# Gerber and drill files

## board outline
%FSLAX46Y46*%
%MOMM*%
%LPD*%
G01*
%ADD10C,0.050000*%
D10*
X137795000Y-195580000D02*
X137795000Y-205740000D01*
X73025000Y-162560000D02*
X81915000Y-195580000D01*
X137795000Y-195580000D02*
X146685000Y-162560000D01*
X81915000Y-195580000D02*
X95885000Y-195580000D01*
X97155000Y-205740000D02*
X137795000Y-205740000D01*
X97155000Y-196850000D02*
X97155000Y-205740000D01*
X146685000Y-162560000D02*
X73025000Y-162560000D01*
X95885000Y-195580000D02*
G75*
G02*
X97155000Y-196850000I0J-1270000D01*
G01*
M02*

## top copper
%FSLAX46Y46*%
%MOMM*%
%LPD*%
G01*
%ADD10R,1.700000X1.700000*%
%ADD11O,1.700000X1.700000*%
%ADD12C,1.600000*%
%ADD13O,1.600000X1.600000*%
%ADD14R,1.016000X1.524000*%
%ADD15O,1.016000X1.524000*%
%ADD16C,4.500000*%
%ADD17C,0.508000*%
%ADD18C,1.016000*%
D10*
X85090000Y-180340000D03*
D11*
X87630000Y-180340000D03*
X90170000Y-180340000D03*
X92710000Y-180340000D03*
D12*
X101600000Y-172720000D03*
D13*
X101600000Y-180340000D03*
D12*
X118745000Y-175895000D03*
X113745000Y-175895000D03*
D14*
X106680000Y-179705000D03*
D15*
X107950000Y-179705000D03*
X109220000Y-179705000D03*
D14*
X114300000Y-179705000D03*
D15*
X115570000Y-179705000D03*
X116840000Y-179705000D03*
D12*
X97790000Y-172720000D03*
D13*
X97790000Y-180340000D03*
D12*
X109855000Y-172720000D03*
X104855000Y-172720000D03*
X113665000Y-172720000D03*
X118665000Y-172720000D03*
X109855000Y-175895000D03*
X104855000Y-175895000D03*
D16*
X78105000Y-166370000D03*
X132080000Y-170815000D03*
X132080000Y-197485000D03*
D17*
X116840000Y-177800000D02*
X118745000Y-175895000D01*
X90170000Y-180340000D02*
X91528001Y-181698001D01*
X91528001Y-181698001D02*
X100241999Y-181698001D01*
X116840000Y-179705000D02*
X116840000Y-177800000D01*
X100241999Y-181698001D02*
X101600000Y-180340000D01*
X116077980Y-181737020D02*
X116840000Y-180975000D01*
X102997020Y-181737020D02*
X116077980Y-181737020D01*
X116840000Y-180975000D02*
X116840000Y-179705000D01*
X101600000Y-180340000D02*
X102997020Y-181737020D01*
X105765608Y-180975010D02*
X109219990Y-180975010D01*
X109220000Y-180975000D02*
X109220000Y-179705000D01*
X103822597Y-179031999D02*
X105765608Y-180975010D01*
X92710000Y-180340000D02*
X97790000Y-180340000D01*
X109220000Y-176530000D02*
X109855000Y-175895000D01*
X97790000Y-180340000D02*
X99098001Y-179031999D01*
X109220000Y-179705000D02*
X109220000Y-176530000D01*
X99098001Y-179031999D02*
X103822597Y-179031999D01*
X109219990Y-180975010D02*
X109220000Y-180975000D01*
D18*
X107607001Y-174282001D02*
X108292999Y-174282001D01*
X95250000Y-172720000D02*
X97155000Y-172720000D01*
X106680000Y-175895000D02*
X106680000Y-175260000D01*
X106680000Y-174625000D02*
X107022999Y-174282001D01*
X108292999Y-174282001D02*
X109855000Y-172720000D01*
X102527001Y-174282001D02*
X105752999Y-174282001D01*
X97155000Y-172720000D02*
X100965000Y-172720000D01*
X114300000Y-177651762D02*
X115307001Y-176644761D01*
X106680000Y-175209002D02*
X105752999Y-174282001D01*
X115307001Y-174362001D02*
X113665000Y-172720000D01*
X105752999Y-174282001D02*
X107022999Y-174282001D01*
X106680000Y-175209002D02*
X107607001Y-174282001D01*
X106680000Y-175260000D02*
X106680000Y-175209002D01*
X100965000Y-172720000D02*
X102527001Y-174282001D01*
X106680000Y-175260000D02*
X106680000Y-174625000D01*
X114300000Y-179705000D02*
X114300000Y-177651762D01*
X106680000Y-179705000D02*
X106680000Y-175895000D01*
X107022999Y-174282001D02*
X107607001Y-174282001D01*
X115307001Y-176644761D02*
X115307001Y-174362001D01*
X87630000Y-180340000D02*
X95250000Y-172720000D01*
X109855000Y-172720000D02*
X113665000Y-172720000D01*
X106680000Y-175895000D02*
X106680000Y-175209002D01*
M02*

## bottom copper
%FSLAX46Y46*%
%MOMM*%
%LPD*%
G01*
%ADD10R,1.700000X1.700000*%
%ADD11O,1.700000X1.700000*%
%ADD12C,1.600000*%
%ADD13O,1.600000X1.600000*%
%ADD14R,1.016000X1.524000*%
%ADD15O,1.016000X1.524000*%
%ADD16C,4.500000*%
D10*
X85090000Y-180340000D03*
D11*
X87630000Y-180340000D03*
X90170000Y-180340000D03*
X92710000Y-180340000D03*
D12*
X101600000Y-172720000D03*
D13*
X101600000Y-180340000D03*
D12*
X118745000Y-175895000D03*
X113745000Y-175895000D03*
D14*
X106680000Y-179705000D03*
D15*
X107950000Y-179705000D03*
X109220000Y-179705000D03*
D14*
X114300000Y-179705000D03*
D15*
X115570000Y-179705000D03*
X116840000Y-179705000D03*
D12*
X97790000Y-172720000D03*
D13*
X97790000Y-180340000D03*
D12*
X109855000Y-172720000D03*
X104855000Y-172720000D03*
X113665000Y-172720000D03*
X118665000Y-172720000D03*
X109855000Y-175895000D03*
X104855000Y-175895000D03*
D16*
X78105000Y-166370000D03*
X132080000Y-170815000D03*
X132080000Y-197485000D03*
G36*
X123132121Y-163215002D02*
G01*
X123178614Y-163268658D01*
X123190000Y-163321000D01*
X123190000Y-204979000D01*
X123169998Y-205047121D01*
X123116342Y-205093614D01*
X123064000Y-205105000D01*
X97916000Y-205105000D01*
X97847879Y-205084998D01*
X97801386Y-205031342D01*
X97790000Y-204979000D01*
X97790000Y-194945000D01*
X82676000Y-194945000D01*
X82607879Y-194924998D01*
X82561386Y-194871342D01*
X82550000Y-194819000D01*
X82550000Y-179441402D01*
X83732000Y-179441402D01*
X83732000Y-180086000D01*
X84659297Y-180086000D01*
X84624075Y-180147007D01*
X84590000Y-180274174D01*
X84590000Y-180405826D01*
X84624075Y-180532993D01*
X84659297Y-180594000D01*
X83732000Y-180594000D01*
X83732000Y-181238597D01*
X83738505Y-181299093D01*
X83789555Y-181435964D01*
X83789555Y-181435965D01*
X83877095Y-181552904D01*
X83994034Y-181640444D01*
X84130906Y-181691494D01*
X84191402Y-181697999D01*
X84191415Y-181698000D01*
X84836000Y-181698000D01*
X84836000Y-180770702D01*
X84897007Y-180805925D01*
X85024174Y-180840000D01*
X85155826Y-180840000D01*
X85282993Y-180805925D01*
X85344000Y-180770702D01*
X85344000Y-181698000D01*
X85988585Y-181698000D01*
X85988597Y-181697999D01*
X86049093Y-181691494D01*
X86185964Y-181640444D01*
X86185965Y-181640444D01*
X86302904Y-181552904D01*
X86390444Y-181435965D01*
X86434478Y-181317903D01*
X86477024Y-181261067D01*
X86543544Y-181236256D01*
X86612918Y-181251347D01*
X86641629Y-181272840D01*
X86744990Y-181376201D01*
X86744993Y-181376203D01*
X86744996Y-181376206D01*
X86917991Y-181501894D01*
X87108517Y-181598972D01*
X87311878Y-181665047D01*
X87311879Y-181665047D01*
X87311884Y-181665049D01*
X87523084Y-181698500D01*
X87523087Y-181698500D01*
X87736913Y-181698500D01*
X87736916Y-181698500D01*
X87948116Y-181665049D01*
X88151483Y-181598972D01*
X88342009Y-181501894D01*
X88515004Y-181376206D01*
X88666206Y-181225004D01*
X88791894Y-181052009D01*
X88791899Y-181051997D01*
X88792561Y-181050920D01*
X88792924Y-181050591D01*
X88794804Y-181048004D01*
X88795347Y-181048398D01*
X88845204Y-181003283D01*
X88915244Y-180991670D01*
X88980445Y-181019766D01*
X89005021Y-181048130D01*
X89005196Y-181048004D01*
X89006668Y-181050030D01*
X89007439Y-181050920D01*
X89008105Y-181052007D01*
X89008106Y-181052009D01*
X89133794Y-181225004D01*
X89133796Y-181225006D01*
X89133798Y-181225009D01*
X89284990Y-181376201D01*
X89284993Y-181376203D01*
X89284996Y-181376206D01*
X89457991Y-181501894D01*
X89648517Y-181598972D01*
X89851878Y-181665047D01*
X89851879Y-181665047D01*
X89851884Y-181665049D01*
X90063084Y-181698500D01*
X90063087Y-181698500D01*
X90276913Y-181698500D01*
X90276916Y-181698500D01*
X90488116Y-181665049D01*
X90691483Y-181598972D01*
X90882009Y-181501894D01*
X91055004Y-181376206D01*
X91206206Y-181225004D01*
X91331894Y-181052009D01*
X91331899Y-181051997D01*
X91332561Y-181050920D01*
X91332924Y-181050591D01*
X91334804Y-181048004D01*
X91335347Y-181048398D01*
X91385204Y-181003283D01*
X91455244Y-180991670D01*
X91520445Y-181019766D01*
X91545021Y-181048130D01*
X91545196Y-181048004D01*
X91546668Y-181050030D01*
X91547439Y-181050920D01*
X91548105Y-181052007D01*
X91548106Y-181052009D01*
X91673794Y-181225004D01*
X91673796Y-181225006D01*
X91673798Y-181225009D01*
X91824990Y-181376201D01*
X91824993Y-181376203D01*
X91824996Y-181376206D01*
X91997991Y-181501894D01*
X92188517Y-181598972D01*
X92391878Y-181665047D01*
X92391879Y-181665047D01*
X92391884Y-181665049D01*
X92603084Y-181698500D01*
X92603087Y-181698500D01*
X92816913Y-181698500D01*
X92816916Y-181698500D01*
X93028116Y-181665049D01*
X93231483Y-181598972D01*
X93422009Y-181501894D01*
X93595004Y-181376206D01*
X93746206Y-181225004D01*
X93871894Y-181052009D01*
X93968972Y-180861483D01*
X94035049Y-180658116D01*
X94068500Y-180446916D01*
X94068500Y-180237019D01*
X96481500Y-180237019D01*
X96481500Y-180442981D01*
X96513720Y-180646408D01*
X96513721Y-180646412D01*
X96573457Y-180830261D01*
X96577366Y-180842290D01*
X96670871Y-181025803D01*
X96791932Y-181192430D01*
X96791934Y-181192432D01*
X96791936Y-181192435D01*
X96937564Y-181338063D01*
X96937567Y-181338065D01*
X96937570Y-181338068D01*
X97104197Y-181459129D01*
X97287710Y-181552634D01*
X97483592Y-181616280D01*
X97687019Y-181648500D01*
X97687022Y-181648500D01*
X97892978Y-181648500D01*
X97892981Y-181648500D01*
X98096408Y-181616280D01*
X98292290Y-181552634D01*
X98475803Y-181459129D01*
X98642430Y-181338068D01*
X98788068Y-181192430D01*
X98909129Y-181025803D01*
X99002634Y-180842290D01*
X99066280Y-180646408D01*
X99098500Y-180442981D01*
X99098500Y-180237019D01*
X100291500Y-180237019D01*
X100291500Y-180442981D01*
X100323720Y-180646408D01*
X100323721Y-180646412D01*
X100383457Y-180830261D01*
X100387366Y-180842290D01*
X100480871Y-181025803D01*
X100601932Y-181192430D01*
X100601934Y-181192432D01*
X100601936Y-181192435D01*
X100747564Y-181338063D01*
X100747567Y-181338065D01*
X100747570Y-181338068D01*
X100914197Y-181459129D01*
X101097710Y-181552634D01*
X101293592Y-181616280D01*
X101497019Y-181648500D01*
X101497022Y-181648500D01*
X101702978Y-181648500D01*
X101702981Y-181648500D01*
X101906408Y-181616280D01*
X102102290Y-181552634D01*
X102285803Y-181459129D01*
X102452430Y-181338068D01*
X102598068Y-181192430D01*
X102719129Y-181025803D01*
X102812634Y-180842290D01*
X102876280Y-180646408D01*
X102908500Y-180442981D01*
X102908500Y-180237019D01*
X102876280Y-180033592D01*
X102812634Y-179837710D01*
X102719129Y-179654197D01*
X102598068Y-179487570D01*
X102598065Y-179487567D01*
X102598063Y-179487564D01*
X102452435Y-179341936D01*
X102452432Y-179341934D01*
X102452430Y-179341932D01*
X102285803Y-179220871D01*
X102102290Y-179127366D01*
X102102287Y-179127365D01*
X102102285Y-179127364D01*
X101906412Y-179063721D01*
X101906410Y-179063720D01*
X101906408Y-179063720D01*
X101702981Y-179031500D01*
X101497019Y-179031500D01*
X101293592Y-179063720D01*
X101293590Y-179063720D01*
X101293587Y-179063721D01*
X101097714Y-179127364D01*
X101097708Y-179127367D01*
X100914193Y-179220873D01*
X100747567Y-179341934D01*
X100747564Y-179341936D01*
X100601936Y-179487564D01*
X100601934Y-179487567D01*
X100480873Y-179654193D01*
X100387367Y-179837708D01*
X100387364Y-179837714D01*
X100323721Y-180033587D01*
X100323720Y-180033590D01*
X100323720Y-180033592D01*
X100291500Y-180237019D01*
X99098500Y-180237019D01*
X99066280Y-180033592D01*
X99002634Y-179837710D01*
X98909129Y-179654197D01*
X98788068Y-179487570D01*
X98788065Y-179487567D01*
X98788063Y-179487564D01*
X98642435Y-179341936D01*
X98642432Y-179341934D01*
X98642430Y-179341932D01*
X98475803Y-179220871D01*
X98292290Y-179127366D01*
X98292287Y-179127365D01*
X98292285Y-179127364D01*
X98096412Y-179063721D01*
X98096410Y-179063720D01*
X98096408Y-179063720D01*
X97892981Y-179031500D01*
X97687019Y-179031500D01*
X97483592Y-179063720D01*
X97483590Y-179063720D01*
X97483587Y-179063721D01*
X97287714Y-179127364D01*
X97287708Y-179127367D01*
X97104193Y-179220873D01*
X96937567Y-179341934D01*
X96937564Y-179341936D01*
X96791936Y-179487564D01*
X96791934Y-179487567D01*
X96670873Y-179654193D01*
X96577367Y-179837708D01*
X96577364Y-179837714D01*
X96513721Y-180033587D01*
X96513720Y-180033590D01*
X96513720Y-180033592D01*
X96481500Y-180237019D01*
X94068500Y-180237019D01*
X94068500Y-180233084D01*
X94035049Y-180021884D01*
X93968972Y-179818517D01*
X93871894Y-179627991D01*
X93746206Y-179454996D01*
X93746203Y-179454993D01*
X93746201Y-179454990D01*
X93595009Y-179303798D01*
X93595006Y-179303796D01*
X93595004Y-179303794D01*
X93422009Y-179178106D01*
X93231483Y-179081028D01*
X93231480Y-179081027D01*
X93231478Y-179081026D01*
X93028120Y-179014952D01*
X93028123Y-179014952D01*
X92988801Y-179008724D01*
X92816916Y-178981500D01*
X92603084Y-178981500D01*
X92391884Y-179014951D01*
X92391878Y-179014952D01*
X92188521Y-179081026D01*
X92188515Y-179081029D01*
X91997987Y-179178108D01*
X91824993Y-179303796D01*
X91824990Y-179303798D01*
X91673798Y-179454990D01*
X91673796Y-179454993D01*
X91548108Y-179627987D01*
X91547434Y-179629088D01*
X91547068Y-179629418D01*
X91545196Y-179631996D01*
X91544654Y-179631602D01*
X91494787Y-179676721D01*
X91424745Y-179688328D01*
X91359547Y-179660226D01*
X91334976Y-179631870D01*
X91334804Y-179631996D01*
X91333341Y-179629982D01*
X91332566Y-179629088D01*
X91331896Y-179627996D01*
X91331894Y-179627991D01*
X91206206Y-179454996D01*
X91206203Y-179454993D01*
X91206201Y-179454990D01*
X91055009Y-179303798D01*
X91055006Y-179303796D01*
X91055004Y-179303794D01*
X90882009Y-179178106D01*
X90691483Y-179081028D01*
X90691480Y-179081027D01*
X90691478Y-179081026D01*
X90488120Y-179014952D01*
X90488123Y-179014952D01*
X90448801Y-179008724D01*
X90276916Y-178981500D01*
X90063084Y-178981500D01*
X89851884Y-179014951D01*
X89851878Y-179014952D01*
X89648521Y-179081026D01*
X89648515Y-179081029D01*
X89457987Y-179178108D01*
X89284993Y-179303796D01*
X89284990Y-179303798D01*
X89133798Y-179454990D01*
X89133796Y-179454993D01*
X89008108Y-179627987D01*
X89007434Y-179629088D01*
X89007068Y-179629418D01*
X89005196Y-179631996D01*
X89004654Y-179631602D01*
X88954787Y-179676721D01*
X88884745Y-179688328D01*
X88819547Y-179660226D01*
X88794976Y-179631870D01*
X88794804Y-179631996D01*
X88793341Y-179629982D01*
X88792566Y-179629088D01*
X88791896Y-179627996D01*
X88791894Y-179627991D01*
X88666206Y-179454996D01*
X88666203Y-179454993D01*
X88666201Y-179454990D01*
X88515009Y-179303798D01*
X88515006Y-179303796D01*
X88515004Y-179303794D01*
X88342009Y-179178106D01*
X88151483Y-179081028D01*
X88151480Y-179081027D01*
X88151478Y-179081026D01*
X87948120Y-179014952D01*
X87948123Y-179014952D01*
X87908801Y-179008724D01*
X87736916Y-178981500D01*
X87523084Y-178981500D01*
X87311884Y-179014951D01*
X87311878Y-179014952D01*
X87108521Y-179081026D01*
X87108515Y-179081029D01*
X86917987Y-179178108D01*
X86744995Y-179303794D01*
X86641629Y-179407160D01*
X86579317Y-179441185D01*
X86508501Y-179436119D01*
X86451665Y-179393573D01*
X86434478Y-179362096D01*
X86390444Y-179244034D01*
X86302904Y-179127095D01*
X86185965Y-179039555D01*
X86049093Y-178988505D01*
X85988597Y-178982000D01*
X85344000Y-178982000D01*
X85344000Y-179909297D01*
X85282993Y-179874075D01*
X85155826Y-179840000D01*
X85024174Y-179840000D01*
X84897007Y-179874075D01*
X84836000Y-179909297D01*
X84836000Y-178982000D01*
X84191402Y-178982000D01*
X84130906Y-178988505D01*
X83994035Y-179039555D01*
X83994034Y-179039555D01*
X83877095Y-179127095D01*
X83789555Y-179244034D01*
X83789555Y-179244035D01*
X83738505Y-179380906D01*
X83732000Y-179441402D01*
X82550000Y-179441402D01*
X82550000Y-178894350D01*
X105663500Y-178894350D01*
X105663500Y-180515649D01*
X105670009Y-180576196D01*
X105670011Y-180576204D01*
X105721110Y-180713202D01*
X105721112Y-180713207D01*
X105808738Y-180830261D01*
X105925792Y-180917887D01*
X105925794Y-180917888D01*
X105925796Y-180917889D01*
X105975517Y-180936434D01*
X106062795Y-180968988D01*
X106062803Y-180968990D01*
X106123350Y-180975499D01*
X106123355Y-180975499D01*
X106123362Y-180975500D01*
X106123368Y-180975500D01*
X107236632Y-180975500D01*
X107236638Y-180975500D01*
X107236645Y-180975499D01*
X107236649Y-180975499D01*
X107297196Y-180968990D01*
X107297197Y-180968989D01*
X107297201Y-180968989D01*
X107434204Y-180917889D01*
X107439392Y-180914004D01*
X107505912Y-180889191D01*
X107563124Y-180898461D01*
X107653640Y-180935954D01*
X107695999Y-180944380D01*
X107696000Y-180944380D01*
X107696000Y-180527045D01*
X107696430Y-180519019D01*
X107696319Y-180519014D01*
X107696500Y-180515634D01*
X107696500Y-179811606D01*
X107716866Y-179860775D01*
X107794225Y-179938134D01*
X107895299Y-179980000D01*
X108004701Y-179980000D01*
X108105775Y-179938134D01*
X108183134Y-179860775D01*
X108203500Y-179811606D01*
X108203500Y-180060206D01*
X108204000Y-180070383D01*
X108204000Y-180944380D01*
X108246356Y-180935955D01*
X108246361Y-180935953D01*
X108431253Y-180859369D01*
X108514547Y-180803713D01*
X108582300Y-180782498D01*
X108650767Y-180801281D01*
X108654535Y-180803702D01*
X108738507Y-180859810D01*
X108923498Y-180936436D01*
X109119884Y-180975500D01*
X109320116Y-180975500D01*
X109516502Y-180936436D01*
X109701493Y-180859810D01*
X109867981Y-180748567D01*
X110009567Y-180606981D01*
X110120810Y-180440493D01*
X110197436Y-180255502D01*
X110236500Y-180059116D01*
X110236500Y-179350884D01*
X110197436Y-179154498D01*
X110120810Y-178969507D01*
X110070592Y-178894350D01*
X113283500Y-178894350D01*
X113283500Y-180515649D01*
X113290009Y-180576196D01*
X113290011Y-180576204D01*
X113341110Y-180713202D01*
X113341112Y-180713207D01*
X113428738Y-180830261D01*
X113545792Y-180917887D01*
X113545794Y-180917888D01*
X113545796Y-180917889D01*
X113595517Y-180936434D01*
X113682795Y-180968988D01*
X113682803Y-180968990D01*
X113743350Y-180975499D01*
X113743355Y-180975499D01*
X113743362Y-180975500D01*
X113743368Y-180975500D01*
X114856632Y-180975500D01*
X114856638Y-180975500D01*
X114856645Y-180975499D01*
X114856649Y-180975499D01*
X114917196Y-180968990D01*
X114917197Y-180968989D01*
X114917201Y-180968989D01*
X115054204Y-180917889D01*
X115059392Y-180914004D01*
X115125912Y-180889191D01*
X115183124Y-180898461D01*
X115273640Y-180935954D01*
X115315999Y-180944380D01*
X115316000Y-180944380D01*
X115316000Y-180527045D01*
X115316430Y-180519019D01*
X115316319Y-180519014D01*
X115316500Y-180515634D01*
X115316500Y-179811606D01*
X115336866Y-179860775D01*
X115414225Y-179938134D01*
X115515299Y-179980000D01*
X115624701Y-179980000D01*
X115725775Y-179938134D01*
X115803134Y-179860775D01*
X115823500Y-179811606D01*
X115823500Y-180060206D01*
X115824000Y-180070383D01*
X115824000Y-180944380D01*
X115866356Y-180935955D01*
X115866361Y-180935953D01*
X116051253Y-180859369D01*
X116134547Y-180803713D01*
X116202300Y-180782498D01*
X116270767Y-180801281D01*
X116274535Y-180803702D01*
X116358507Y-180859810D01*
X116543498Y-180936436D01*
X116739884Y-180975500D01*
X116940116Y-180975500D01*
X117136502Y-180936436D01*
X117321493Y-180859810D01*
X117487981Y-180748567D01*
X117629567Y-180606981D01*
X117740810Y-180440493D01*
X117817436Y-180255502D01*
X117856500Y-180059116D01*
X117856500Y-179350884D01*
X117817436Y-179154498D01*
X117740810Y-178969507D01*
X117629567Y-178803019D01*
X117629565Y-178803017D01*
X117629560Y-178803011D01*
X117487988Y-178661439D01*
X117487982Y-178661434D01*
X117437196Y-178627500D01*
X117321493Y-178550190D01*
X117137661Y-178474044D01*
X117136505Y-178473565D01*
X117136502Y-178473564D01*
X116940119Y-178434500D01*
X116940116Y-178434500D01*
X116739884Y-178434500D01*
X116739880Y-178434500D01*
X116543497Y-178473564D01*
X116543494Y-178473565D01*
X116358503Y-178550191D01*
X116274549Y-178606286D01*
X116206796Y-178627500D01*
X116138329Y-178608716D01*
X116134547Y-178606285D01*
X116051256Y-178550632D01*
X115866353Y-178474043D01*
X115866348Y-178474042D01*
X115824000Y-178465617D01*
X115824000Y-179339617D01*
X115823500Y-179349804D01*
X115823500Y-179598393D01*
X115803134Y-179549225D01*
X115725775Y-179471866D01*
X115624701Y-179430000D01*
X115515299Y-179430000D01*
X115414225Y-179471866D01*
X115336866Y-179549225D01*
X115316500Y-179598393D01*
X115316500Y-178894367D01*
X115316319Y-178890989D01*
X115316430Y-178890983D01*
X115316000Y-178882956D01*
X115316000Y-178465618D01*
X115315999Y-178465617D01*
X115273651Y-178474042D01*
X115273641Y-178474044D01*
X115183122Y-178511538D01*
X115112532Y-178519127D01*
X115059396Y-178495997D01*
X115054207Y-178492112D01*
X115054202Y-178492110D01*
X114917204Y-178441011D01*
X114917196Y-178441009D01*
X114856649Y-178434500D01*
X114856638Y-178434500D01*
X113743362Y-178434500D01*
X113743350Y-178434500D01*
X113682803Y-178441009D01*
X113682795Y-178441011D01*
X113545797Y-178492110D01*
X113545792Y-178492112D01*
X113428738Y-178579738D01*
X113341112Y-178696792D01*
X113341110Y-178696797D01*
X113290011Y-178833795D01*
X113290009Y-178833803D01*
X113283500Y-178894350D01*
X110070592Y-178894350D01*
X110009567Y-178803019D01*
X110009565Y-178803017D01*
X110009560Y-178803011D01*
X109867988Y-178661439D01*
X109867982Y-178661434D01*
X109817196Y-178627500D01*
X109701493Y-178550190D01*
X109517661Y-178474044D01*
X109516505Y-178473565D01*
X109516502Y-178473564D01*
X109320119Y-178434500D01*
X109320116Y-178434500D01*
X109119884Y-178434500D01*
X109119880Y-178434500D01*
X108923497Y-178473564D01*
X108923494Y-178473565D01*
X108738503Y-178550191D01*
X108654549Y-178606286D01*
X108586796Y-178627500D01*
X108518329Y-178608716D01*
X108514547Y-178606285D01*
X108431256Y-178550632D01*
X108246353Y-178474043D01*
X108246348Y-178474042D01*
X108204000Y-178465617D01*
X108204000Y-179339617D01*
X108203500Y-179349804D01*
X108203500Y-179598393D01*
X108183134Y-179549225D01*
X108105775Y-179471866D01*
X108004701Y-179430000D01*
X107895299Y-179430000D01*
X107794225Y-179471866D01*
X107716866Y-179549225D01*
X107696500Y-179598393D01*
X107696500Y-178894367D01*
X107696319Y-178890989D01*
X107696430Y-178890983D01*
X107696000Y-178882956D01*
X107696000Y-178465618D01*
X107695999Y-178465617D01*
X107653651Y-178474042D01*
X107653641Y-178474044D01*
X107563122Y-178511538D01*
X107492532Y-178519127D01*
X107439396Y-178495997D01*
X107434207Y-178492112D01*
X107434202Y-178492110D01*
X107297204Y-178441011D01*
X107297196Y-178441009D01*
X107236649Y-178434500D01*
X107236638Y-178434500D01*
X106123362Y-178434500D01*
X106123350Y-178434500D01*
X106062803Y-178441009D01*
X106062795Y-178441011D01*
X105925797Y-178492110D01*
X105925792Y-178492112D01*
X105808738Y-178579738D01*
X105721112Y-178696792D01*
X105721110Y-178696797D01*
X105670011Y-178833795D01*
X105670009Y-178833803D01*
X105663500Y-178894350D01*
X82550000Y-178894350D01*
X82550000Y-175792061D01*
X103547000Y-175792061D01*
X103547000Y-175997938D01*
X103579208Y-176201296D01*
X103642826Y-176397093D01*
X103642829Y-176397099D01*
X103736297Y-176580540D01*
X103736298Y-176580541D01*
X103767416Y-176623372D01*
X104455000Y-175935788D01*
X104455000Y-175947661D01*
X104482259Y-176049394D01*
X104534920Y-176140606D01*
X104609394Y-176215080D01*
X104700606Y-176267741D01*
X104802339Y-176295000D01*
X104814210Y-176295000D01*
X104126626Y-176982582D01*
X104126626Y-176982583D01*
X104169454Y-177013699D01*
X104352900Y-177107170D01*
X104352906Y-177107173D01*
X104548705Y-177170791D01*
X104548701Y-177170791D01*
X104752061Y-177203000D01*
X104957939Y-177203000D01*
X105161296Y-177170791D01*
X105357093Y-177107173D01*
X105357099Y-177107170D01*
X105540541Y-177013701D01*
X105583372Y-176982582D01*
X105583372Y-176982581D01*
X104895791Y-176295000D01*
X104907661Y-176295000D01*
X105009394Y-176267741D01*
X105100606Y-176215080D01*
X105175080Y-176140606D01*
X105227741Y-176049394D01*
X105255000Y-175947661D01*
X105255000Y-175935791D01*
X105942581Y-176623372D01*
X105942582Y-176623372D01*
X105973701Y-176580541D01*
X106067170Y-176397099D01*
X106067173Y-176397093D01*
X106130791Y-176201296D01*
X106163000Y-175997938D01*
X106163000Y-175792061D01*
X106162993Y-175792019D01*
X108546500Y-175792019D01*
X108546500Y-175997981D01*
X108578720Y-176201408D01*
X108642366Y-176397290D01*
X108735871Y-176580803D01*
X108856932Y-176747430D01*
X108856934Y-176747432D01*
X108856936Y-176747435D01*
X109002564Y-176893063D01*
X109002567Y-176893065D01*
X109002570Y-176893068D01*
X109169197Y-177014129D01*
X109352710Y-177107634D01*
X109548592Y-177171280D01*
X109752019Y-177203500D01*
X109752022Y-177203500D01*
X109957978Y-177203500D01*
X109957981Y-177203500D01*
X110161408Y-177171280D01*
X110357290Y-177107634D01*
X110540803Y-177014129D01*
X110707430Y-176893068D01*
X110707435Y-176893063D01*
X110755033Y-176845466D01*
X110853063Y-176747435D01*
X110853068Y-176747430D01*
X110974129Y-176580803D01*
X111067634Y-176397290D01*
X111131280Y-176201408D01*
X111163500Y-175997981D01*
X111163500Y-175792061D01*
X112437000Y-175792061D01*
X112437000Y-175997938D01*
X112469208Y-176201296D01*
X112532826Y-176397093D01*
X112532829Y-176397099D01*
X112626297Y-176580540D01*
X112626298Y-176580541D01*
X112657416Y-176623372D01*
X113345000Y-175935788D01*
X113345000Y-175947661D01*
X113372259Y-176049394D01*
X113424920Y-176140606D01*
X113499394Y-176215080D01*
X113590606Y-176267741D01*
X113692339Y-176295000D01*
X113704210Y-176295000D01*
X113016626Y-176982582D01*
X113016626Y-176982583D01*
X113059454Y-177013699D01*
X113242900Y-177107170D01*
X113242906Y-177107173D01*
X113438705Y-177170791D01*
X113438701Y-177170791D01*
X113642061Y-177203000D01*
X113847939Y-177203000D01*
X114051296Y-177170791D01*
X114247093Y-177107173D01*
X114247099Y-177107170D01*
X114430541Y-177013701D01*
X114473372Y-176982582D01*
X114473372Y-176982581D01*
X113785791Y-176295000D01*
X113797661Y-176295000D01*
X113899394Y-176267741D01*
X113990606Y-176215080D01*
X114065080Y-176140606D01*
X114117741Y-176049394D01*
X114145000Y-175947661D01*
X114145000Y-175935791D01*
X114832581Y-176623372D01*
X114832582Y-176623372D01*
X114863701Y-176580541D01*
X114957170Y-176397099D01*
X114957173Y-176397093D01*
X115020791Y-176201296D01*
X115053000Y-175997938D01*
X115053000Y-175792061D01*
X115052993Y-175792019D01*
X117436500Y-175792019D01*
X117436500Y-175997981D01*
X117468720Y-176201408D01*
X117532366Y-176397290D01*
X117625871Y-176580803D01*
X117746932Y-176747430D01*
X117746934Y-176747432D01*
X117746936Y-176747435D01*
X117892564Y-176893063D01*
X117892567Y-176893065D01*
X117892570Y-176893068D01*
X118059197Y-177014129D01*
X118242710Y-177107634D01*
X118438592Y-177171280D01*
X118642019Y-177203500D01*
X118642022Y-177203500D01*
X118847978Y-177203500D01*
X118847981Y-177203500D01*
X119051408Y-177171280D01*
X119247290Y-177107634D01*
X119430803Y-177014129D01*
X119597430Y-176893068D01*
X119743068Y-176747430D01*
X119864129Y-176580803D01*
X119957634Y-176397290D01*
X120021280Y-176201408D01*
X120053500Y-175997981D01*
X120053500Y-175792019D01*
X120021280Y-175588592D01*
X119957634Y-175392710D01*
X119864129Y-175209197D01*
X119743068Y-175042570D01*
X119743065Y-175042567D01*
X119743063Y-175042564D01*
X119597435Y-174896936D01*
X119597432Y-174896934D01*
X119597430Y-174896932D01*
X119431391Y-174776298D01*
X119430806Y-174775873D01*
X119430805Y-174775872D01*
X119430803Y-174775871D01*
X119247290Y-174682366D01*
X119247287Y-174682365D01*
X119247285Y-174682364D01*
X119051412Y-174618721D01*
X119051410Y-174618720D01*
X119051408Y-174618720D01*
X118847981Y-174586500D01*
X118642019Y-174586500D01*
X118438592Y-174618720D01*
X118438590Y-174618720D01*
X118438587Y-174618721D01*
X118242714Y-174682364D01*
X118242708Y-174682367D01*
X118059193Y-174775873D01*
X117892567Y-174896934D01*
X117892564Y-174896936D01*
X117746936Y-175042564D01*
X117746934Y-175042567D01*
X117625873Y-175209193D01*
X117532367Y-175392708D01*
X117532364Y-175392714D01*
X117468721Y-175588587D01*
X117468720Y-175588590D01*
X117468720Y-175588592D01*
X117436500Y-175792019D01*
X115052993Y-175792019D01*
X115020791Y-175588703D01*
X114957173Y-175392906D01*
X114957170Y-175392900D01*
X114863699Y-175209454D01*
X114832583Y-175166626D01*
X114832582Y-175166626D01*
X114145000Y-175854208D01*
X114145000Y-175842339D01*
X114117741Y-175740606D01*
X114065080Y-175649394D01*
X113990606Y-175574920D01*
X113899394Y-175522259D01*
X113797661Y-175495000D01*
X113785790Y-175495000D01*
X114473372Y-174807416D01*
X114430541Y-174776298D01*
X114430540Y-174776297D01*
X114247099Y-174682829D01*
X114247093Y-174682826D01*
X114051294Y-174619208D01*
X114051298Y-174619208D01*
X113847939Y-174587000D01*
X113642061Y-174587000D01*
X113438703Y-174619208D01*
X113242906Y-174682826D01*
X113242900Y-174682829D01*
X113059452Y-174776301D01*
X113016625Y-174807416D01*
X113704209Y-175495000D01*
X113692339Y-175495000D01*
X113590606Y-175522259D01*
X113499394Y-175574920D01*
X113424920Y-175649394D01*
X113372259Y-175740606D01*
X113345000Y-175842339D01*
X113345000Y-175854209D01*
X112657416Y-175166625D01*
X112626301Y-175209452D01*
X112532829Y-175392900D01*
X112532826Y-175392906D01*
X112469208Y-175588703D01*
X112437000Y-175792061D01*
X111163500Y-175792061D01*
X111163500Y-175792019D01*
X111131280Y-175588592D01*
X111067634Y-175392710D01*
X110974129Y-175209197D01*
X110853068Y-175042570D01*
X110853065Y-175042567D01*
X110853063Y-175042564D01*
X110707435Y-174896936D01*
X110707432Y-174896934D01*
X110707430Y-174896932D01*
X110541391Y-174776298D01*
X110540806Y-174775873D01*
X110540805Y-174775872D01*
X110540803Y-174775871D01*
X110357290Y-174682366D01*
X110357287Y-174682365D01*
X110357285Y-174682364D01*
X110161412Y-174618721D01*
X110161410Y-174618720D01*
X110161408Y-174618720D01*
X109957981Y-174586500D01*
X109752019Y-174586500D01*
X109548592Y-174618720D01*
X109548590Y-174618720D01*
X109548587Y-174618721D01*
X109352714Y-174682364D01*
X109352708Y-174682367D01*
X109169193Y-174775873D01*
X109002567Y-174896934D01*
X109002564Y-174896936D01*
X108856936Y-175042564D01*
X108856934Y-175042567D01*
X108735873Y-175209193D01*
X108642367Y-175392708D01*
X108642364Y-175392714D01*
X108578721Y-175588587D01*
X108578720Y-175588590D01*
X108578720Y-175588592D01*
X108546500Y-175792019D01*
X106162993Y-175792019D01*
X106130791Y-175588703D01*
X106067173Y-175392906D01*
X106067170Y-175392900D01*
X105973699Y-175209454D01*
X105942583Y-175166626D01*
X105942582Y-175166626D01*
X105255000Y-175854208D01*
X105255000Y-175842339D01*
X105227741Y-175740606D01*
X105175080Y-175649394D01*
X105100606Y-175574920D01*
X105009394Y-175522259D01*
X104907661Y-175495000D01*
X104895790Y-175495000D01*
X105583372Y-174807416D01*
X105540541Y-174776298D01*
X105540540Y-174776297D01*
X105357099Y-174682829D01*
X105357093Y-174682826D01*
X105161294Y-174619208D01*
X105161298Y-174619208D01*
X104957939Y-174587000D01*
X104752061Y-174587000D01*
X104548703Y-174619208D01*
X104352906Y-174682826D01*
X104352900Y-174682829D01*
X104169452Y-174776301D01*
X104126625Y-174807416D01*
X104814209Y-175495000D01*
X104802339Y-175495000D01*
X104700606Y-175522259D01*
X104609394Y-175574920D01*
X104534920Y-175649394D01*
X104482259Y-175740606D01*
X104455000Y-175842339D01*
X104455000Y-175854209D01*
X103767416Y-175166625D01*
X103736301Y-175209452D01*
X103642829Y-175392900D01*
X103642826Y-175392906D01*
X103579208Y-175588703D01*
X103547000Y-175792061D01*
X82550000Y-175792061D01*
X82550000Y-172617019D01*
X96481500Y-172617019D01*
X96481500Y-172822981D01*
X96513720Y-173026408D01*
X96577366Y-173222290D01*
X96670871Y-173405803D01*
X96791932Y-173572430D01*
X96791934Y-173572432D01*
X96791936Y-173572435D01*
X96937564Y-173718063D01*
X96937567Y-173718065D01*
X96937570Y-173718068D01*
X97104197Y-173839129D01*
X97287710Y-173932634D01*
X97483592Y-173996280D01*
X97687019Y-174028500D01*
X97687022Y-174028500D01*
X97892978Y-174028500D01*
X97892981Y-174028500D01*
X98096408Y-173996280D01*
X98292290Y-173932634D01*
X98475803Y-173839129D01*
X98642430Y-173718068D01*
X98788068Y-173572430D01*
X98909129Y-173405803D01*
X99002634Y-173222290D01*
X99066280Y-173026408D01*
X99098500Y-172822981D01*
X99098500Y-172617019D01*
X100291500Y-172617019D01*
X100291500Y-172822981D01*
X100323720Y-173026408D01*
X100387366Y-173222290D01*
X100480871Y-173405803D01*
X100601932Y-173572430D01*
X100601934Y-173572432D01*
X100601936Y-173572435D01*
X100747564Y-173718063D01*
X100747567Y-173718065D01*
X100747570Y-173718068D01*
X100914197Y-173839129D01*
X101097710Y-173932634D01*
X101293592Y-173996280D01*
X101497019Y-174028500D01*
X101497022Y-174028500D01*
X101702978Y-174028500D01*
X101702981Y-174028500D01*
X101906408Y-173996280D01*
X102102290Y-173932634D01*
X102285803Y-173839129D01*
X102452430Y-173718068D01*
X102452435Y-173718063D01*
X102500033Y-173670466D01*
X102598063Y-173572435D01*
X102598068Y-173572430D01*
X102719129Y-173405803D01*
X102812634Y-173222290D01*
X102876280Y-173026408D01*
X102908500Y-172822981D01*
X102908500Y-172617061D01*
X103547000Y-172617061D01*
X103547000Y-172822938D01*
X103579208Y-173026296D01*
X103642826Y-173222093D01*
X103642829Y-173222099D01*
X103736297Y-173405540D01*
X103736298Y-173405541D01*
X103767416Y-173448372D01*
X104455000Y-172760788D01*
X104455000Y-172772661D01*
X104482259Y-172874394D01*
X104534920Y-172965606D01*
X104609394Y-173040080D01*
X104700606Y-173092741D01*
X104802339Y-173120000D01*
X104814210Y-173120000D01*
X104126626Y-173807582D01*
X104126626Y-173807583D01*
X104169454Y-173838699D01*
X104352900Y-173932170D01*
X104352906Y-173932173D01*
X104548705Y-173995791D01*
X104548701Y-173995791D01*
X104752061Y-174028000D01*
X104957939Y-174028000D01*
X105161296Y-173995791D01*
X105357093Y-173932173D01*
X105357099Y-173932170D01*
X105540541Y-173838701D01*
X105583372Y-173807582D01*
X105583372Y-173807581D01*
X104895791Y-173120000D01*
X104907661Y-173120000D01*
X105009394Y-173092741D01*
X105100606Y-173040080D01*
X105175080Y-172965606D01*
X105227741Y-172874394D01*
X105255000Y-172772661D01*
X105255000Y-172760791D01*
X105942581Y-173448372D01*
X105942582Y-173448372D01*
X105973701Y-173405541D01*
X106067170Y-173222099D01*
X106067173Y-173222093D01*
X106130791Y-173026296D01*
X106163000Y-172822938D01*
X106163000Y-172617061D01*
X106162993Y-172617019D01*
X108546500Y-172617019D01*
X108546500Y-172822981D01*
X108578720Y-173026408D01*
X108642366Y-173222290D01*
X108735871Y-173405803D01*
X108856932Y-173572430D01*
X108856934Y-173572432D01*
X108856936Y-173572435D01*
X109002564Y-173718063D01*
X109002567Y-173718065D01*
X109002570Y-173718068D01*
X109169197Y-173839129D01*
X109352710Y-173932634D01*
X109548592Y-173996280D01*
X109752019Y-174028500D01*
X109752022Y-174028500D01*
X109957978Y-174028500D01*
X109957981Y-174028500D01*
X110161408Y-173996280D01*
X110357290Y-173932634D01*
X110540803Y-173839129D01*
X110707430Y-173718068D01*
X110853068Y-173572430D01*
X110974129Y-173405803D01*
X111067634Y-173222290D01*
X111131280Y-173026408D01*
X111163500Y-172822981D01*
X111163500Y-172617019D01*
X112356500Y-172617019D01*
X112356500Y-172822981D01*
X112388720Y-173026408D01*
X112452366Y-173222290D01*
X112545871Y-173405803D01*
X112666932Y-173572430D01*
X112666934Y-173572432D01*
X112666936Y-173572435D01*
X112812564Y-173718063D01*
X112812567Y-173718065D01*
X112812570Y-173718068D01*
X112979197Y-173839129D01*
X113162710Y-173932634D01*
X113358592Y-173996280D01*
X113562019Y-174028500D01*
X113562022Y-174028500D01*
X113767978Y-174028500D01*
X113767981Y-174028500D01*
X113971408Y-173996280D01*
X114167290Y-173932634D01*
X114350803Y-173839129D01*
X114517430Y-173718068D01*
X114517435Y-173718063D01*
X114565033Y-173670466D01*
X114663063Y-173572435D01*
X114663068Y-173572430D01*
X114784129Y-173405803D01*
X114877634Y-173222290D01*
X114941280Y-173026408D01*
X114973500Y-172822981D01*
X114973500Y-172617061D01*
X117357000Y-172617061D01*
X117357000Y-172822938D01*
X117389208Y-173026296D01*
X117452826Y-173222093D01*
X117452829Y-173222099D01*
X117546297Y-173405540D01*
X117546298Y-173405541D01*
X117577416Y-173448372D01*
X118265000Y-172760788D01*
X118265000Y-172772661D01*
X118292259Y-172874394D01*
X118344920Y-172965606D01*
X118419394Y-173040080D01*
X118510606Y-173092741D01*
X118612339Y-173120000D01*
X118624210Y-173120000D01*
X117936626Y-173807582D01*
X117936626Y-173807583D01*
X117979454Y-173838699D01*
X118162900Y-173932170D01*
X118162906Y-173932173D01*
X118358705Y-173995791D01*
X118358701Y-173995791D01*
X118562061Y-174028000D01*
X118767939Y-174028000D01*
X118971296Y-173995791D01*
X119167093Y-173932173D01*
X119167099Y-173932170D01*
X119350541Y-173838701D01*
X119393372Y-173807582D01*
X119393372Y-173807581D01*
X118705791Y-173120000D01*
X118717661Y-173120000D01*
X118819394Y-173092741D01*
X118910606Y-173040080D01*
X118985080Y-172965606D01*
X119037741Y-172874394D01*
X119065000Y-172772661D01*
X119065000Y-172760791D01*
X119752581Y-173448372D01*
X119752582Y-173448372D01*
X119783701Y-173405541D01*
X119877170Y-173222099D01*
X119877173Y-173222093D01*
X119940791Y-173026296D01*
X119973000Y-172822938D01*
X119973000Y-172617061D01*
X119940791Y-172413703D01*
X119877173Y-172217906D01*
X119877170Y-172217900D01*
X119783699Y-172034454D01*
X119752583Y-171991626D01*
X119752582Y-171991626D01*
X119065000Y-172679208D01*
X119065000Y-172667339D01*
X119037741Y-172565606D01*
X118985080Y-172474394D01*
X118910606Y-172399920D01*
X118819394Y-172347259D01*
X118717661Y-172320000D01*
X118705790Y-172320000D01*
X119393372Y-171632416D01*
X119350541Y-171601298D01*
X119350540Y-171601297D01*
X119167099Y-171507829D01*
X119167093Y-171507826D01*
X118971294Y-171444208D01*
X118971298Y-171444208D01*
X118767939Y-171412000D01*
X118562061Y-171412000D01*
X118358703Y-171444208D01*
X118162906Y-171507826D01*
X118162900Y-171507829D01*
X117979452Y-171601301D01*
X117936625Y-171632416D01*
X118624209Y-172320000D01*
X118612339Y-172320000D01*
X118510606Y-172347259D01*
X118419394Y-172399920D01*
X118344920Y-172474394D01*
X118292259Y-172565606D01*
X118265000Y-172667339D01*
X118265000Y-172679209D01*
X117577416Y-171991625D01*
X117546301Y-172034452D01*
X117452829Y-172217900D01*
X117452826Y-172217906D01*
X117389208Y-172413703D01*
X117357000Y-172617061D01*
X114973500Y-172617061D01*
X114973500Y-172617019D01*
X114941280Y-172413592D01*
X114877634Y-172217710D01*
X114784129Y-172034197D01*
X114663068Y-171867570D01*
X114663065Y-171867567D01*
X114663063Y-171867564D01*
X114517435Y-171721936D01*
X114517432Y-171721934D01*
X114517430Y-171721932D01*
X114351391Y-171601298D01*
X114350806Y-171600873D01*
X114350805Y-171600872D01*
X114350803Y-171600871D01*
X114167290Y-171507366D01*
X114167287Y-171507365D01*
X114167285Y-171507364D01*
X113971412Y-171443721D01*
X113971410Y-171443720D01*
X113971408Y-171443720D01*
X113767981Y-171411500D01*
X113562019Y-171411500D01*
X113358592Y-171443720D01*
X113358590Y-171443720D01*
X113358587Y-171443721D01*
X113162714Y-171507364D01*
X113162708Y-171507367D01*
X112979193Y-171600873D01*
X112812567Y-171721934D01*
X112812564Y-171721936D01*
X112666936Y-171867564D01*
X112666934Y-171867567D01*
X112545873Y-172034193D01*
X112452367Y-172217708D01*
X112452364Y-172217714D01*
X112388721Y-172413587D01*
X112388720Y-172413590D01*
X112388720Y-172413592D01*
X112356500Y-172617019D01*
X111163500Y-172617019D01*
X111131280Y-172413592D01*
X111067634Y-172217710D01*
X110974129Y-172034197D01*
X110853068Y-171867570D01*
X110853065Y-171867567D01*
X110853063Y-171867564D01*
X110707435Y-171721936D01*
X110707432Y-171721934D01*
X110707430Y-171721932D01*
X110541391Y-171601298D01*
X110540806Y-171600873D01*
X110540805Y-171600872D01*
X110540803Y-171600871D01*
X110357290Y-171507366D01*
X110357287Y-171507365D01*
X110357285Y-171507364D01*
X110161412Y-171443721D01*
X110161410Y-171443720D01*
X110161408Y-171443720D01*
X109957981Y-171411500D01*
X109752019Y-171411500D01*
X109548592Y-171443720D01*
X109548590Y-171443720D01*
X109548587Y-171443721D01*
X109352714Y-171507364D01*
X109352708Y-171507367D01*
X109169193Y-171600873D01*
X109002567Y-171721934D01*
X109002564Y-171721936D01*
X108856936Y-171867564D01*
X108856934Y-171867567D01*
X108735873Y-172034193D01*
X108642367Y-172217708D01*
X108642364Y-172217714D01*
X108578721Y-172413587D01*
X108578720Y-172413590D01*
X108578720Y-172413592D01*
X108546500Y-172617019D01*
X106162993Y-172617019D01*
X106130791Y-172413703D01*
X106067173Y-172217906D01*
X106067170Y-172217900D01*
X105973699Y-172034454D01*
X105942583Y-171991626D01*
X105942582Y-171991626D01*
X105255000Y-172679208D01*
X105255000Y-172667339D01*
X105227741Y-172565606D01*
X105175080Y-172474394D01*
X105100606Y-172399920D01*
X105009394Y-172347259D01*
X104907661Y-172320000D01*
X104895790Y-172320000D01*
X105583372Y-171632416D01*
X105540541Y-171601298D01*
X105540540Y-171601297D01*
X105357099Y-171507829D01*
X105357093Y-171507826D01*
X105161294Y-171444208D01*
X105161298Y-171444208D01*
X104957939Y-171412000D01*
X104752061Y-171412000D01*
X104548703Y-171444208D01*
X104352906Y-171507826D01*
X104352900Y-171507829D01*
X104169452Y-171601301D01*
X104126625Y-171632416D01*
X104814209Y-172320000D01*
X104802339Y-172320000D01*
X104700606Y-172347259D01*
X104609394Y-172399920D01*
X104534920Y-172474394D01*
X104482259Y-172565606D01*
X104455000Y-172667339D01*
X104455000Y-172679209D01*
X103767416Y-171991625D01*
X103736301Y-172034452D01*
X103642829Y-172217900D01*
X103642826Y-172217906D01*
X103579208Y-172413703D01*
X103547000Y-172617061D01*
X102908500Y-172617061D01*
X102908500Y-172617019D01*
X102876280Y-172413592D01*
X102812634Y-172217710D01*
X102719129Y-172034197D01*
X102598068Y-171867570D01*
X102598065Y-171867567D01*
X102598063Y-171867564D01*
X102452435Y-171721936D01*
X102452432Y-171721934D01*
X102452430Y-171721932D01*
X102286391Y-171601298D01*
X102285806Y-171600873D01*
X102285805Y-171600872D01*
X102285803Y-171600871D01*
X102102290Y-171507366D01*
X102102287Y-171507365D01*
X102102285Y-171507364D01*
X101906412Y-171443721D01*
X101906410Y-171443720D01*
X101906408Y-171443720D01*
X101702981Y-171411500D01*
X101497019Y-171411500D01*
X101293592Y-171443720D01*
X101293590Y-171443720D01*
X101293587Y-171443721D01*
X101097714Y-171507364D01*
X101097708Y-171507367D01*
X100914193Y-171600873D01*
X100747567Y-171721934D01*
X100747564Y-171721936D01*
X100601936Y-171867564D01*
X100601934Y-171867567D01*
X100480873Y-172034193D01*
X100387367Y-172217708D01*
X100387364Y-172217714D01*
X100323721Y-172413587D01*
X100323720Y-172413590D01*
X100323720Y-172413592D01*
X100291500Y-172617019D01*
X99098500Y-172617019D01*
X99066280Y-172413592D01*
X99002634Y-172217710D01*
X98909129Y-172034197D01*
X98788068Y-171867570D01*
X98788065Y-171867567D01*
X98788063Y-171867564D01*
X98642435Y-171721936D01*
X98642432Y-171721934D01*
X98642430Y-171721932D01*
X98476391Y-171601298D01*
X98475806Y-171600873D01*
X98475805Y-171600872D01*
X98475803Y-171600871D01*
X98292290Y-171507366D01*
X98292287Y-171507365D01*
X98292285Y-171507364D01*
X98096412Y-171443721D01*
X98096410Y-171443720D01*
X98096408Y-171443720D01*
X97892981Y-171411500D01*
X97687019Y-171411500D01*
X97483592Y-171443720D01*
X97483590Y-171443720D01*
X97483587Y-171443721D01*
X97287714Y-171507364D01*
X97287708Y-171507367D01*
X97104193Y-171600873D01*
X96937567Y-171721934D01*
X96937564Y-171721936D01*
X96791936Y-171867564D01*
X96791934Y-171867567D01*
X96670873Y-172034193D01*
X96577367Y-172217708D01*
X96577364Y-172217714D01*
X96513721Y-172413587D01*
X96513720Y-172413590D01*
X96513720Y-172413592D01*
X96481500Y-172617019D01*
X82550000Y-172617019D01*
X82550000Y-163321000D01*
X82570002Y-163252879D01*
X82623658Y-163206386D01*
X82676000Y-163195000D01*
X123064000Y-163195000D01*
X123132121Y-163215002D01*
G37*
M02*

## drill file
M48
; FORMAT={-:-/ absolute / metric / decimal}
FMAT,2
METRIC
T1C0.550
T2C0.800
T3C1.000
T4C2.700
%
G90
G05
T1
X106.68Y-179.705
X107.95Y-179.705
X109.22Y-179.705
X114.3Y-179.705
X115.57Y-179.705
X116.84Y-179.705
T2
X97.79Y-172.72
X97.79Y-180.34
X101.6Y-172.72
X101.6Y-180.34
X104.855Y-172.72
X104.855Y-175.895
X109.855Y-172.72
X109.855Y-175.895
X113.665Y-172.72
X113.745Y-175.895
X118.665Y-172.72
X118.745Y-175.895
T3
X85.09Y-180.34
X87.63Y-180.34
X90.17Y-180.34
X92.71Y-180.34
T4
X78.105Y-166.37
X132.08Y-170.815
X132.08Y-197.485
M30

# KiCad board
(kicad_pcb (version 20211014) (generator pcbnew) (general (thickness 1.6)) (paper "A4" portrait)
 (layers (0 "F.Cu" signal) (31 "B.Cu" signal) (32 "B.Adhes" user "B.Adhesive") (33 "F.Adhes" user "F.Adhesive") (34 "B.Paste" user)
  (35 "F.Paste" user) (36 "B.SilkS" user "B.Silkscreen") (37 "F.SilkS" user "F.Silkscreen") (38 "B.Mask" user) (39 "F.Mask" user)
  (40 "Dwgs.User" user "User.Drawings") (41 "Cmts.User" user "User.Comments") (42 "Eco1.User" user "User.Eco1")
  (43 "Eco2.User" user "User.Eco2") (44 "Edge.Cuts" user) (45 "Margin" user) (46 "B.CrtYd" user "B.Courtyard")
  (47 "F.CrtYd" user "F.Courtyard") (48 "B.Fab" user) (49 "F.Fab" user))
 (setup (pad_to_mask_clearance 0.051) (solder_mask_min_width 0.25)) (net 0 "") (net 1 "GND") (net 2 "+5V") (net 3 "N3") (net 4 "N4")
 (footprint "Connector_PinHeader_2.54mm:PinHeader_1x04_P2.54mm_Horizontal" (layer "F.Cu") (at 85.09 180.34 90)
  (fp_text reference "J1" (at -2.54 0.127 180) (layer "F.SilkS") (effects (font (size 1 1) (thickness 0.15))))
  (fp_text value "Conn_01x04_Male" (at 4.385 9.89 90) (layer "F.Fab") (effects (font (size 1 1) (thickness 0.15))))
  (pad "1" thru_hole rect locked (at 0 0 90) (size 1.7 1.7) (drill 1) (layers *.Cu *.Mask) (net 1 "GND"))
  (pad "2" thru_hole oval locked (at 0 2.54 90) (size 1.7 1.7) (drill 1) (layers *.Cu *.Mask) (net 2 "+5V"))
  (pad "3" thru_hole oval locked (at 0 5.08 90) (size 1.7 1.7) (drill 1) (layers *.Cu *.Mask) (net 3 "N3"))
  (pad "4" thru_hole oval locked (at 0 7.62 90) (size 1.7 1.7) (drill 1) (layers *.Cu *.Mask) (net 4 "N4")))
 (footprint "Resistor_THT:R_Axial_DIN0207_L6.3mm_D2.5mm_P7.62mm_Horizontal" (layer "F.Cu") (at 101.6 172.72 -90)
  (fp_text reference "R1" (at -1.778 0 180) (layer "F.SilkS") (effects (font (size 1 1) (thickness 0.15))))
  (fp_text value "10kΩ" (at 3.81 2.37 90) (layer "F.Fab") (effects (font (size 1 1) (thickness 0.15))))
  (pad "1" thru_hole circle locked (at 0 0 270) (size 1.6 1.6) (drill 0.8) (layers *.Cu *.Mask) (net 2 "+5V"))
  (pad "2" thru_hole oval locked (at 7.62 0 270) (size 1.6 1.6) (drill 0.8) (layers *.Cu *.Mask) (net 3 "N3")))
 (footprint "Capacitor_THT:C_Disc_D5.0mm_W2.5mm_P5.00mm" (layer "F.Cu") (at 118.745 175.895 180)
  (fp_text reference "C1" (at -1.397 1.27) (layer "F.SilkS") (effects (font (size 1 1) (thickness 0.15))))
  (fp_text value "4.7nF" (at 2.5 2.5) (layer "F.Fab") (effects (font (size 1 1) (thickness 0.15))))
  (pad "1" thru_hole circle locked (at 0 0 180) (size 1.6 1.6) (drill 0.8) (layers *.Cu *.Mask) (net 3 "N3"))
  (pad "2" thru_hole circle locked (at 5 0 180) (size 1.6 1.6) (drill 0.8) (layers *.Cu *.Mask) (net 1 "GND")))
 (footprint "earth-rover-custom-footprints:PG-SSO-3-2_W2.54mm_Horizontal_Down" (layer "F.Cu") (at 106.68 179.705 90)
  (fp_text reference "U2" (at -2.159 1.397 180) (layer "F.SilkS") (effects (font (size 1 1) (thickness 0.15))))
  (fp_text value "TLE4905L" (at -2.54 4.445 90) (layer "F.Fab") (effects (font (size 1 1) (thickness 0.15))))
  (pad "1" thru_hole rect locked (at 0 0 90) (size 1.524 1.016) (drill 0.55) (layers *.Cu *.Mask) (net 2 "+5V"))
  (pad "2" thru_hole oval locked (at 0 1.27 90) (size 1.524 1.016) (drill 0.55) (layers *.Cu *.Mask) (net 1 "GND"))
  (pad "3" thru_hole oval locked (at 0 2.54 90) (size 1.524 1.016) (drill 0.55) (layers *.Cu *.Mask) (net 4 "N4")))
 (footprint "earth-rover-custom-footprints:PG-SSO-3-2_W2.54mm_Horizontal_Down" (layer "F.Cu") (at 114.3 179.705 90)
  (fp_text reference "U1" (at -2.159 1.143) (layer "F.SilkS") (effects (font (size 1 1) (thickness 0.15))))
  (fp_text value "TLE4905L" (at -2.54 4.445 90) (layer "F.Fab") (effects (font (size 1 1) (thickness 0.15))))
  (pad "1" thru_hole rect locked (at 0 0 90) (size 1.524 1.016) (drill 0.55) (layers *.Cu *.Mask) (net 2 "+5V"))
  (pad "2" thru_hole oval locked (at 0 1.27 90) (size 1.524 1.016) (drill 0.55) (layers *.Cu *.Mask) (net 1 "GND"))
  (pad "3" thru_hole oval locked (at 0 2.54 90) (size 1.524 1.016) (drill 0.55) (layers *.Cu *.Mask) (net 3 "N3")))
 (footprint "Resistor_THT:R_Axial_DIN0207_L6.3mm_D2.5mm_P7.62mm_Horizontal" (layer "F.Cu") (at 97.79 172.72 -90)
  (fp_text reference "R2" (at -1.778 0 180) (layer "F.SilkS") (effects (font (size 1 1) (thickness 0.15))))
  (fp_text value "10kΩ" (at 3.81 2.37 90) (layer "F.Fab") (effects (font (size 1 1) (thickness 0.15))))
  (pad "1" thru_hole circle locked (at 0 0 270) (size 1.6 1.6) (drill 0.8) (layers *.Cu *.Mask) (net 2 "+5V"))
  (pad "2" thru_hole oval locked (at 7.62 0 270) (size 1.6 1.6) (drill 0.8) (layers *.Cu *.Mask) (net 4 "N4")))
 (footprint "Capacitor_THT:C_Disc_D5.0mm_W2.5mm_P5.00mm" (layer "F.Cu") (at 109.855 172.72 180)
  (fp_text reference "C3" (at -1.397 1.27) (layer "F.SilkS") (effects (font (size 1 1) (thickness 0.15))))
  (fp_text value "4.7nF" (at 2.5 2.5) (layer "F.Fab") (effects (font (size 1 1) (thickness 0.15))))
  (pad "1" thru_hole circle locked (at 0 0 180) (size 1.6 1.6) (drill 0.8) (layers *.Cu *.Mask) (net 2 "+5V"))
  (pad "2" thru_hole circle locked (at 5 0 180) (size 1.6 1.6) (drill 0.8) (layers *.Cu *.Mask) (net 1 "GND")))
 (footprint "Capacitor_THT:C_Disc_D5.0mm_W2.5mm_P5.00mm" (layer "F.Cu") (at 113.665 172.72)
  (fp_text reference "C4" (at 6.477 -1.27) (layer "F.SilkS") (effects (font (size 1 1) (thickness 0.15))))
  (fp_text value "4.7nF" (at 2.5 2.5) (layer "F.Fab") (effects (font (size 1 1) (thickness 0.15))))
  (pad "1" thru_hole circle locked (at 0 0) (size 1.6 1.6) (drill 0.8) (layers *.Cu *.Mask) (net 2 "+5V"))
  (pad "2" thru_hole circle locked (at 5 0) (size 1.6 1.6) (drill 0.8) (layers *.Cu *.Mask) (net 1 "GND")))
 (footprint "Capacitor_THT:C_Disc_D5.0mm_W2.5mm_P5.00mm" (layer "F.Cu") (at 109.855 175.895 180)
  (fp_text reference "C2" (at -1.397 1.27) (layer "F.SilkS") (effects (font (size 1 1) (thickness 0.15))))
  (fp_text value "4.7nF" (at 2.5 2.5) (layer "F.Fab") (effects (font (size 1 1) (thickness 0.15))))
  (pad "1" thru_hole circle locked (at 0 0 180) (size 1.6 1.6) (drill 0.8) (layers *.Cu *.Mask) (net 4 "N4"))
  (pad "2" thru_hole circle locked (at 5 0 180) (size 1.6 1.6) (drill 0.8) (layers *.Cu *.Mask) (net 1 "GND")))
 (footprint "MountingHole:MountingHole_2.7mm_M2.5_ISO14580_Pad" (layer "F.Cu") (at 78.105 166.37)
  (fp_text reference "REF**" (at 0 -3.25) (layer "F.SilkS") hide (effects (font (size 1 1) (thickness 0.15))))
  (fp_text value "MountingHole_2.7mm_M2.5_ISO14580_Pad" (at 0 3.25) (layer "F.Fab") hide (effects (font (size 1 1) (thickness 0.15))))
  (pad "1" thru_hole circle locked (at 0 0) (size 4.5 4.5) (drill 2.7) (layers *.Cu *.Mask)))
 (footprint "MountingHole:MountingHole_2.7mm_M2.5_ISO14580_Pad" (layer "F.Cu") (at 132.08 170.815)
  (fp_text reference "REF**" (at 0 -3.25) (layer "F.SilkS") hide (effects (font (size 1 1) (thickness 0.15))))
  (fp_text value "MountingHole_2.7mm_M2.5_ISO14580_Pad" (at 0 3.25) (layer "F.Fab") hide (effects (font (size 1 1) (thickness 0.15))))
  (pad "1" thru_hole circle locked (at 0 0) (size 4.5 4.5) (drill 2.7) (layers *.Cu *.Mask)))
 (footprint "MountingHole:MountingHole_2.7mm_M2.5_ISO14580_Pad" (layer "F.Cu") (at 132.08 197.485)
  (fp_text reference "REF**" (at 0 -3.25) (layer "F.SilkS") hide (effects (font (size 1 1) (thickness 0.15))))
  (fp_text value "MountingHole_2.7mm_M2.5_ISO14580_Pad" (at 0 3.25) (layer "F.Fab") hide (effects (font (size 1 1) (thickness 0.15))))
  (pad "1" thru_hole circle locked (at 0 0) (size 4.5 4.5) (drill 2.7) (layers *.Cu *.Mask)))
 (gr_line (start 137.795 195.58) (end 137.795 205.74) (layer "Edge.Cuts") (width 0.05))
 (gr_line (start 73.025 162.56) (end 81.915 195.58) (layer "Edge.Cuts") (width 0.05))
 (gr_line (start 137.795 195.58) (end 146.685 162.56) (layer "Edge.Cuts") (width 0.05))
 (gr_line (start 81.915 195.58) (end 95.885 195.58) (layer "Edge.Cuts") (width 0.05))
 (gr_line (start 97.155 205.74) (end 137.795 205.74) (layer "Edge.Cuts") (width 0.05))
 (gr_line (start 97.155 196.85) (end 97.155 205.74) (layer "Edge.Cuts") (width 0.05))
 (gr_line (start 146.685 162.56) (end 73.025 162.56) (layer "Edge.Cuts") (width 0.05))
 (gr_arc (start 95.885 195.58) (mid 96.783026 195.951974) (end 97.155 196.85) (layer "Edge.Cuts") (width 0.05))
 (segment (start 116.84 177.8) (end 118.745 175.895) (width 0.508) (layer "F.Cu") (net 3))
 (segment (start 90.17 180.34) (end 91.528001 181.698001) (width 0.508) (layer "F.Cu") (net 3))
 (segment (start 91.528001 181.698001) (end 100.241999 181.698001) (width 0.508) (layer "F.Cu") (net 3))
 (segment (start 116.84 179.705) (end 116.84 177.8) (width 0.508) (layer "F.Cu") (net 3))
 (segment (start 100.241999 181.698001) (end 101.6 180.34) (width 0.508) (layer "F.Cu") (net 3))
 (segment (start 116.07798 181.73702) (end 116.84 180.975) (width 0.508) (layer "F.Cu") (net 3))
 (segment (start 102.99702 181.73702) (end 116.07798 181.73702) (width 0.508) (layer "F.Cu") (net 3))
 (segment (start 116.84 180.975) (end 116.84 179.705) (width 0.508) (layer "F.Cu") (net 3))
 (segment (start 101.6 180.34) (end 102.99702 181.73702) (width 0.508) (layer "F.Cu") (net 3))
 (segment (start 105.765608 180.97501) (end 109.21999 180.97501) (width 0.508) (layer "F.Cu") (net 4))
 (segment (start 109.22 180.975) (end 109.22 179.705) (width 0.508) (layer "F.Cu") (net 4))
 (segment (start 103.822597 179.031999) (end 105.765608 180.97501) (width 0.508) (layer "F.Cu") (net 4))
 (segment (start 92.71 180.34) (end 97.79 180.34) (width 0.508) (layer "F.Cu") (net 4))
 (segment (start 109.22 176.53) (end 109.855 175.895) (width 0.508) (layer "F.Cu") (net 4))
 (segment (start 97.79 180.34) (end 99.098001 179.031999) (width 0.508) (layer "F.Cu") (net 4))
 (segment (start 109.22 179.705) (end 109.22 176.53) (width 0.508) (layer "F.Cu") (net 4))
 (segment (start 99.098001 179.031999) (end 103.822597 179.031999) (width 0.508) (layer "F.Cu") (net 4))
 (segment (start 109.21999 180.97501) (end 109.22 180.975) (width 0.508) (layer "F.Cu") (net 4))
 (segment (start 107.607001 174.282001) (end 108.292999 174.282001) (width 1.016) (layer "F.Cu") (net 2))
 (segment (start 95.25 172.72) (end 97.155 172.72) (width 1.016) (layer "F.Cu") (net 2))
 (segment (start 106.68 175.895) (end 106.68 175.26) (width 1.016) (layer "F.Cu") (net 2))
 (segment (start 106.68 174.625) (end 107.022999 174.282001) (width 1.016) (layer "F.Cu") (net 2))
 (segment (start 108.292999 174.282001) (end 109.855 172.72) (width 1.016) (layer "F.Cu") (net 2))
 (segment (start 102.527001 174.282001) (end 105.752999 174.282001) (width 1.016) (layer "F.Cu") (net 2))
 (segment (start 97.155 172.72) (end 100.965 172.72) (width 1.016) (layer "F.Cu") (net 2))
 (segment (start 114.3 177.651762) (end 115.307001 176.644761) (width 1.016) (layer "F.Cu") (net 2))
 (segment (start 106.68 175.209002) (end 105.752999 174.282001) (width 1.016) (layer "F.Cu") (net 2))
 (segment (start 115.307001 174.362001) (end 113.665 172.72) (width 1.016) (layer "F.Cu") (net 2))
 (segment (start 105.752999 174.282001) (end 107.022999 174.282001) (width 1.016) (layer "F.Cu") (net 2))
 (segment (start 106.68 175.209002) (end 107.607001 174.282001) (width 1.016) (layer "F.Cu") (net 2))
 (segment (start 106.68 175.26) (end 106.68 175.209002) (width 1.016) (layer "F.Cu") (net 2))
 (segment (start 100.965 172.72) (end 102.527001 174.282001) (width 1.016) (layer "F.Cu") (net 2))
 (segment (start 106.68 175.26) (end 106.68 174.625) (width 1.016) (layer "F.Cu") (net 2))
 (segment (start 114.3 179.705) (end 114.3 177.651762) (width 1.016) (layer "F.Cu") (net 2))
 (segment (start 106.68 179.705) (end 106.68 175.895) (width 1.016) (layer "F.Cu") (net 2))
 (segment (start 107.022999 174.282001) (end 107.607001 174.282001) (width 1.016) (layer "F.Cu") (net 2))
 (segment (start 115.307001 176.644761) (end 115.307001 174.362001) (width 1.016) (layer "F.Cu") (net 2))
 (segment (start 87.63 180.34) (end 95.25 172.72) (width 1.016) (layer "F.Cu") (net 2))
 (segment (start 109.855 172.72) (end 113.665 172.72) (width 1.016) (layer "F.Cu") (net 2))
 (segment (start 106.68 175.895) (end 106.68 175.209002) (width 1.016) (layer "F.Cu") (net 2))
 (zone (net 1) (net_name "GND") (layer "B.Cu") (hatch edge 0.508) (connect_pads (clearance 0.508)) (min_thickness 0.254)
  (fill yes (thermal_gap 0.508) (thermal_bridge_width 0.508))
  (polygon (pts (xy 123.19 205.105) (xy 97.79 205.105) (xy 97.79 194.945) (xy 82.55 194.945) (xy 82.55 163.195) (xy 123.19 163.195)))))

